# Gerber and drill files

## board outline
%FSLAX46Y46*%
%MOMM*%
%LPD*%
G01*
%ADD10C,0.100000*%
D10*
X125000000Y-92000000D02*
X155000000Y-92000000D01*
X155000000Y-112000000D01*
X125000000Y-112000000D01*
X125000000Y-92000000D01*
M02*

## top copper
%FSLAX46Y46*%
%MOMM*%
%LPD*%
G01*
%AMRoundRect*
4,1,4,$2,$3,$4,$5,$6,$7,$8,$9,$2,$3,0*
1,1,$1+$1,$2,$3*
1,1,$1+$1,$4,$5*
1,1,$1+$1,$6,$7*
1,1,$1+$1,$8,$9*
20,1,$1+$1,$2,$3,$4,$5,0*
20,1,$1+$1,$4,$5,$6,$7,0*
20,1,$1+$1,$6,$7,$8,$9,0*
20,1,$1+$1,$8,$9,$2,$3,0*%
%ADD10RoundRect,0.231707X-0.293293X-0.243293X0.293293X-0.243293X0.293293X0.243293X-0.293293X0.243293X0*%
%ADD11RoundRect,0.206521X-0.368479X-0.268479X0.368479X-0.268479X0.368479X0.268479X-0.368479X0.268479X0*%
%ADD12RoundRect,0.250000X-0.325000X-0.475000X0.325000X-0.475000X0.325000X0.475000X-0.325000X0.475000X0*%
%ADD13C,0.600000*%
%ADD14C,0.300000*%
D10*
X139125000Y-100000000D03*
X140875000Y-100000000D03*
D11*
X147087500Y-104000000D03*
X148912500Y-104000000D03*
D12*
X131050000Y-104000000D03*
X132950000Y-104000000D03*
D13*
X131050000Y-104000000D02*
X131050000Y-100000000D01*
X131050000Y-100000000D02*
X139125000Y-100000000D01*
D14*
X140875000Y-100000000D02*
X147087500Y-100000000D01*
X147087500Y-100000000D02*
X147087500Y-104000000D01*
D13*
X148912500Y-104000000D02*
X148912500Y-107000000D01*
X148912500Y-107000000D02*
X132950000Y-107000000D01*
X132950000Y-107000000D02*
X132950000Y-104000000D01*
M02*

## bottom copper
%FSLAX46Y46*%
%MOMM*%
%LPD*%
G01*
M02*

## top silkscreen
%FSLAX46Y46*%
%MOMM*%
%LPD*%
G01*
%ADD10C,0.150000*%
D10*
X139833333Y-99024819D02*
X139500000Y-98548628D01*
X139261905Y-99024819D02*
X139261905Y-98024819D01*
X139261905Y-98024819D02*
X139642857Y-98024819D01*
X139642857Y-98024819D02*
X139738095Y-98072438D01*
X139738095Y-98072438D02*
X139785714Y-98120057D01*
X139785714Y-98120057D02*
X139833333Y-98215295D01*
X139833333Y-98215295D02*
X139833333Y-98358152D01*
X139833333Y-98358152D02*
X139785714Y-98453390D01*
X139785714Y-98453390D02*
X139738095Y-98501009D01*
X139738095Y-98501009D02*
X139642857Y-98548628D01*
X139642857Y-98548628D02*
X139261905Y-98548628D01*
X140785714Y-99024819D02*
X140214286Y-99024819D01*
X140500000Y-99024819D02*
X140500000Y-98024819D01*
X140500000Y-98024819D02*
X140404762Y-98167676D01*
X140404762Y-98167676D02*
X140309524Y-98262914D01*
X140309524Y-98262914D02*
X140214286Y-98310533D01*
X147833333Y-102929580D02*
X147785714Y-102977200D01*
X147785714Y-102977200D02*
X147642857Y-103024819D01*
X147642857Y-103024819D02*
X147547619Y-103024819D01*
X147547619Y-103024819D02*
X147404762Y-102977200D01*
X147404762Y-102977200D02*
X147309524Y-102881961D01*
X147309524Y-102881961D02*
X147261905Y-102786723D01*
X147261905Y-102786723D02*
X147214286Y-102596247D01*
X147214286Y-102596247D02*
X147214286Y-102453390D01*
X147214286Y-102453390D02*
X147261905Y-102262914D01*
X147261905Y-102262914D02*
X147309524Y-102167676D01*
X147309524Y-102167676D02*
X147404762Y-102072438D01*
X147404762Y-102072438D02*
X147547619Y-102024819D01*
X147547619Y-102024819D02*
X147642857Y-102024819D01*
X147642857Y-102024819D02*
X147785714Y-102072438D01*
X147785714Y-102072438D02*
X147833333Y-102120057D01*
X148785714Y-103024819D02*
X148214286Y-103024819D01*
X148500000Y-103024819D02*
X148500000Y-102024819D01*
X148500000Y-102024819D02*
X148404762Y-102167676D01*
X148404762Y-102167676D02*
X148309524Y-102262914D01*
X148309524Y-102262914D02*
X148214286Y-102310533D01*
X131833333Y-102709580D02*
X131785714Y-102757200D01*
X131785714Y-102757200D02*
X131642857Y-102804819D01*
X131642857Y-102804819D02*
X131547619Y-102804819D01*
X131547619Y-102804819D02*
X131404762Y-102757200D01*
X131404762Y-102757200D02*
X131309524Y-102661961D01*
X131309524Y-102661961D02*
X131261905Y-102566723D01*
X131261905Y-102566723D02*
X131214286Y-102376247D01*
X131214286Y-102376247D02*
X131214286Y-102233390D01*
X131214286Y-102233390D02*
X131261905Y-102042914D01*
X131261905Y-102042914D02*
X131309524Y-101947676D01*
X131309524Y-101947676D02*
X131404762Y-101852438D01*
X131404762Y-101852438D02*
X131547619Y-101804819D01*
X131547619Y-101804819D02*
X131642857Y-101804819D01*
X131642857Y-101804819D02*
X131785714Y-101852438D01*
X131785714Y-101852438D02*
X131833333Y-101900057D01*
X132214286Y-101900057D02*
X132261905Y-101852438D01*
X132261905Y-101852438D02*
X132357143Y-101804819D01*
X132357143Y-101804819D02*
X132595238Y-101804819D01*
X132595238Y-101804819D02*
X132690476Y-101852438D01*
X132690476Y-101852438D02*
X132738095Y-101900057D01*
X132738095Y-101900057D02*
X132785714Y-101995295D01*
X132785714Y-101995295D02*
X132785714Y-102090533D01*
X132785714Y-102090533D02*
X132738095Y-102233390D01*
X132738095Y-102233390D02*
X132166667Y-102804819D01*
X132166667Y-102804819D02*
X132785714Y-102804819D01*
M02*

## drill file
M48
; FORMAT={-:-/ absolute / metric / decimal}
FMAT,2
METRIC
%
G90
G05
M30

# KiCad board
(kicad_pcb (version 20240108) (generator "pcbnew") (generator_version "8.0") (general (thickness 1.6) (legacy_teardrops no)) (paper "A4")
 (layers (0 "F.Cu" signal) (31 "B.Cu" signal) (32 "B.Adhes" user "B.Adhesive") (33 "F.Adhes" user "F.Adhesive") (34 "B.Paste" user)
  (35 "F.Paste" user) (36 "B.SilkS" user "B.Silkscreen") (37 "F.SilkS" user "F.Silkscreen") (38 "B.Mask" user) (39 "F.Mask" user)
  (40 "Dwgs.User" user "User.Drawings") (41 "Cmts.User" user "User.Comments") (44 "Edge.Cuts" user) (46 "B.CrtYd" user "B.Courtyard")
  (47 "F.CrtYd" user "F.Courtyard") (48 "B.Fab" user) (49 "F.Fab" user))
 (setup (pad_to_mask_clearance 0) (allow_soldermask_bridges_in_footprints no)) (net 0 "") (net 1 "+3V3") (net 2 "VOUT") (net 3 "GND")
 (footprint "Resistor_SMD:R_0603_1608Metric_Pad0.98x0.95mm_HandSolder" (layer "F.Cu") (at 140 100 0)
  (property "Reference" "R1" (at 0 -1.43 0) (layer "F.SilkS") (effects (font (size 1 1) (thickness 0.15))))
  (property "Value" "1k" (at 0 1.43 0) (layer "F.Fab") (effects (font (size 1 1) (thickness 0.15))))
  (pad "1" smd roundrect (at -0.875 0 0) (size 1.05 0.95) (layers "F.Cu" "F.Paste" "F.Mask") (roundrect_rratio 0.243902) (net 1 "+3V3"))
  (pad "2" smd roundrect (at 0.875 0 0) (size 1.05 0.95) (layers "F.Cu" "F.Paste" "F.Mask") (roundrect_rratio 0.243902) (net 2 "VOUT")))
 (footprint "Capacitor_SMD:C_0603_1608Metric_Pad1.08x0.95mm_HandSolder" (layer "F.Cu") (at 148 104)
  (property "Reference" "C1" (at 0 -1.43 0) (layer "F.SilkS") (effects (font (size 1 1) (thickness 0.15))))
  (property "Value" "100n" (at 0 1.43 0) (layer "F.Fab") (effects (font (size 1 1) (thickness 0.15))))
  (pad "1" smd roundrect (at -0.9125 0) (size 1.15 0.95) (layers "F.Cu" "F.Paste" "F.Mask") (roundrect_rratio 0.217391) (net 2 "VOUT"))
  (pad "2" smd roundrect (at 0.9125 0) (size 1.15 0.95) (layers "F.Cu" "F.Paste" "F.Mask") (roundrect_rratio 0.217391) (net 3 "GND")))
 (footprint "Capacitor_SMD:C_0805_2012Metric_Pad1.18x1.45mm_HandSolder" (layer "F.Cu") (at 132 104)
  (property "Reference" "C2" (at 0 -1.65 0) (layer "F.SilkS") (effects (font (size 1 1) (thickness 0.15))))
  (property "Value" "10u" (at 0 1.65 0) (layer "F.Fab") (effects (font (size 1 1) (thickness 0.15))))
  (pad "1" smd roundrect (at -0.95 0) (size 1.15 1.45) (layers "F.Cu" "F.Paste" "F.Mask") (roundrect_rratio 0.217391) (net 1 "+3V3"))
  (pad "2" smd roundrect (at 0.95 0) (size 1.15 1.45) (layers "F.Cu" "F.Paste" "F.Mask") (roundrect_rratio 0.217391) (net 3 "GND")))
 (gr_rect (start 125 92) (end 155 112) (stroke (width 0.1) (type default)) (fill none) (layer "Edge.Cuts"))
 (segment (start 131.05 104) (end 131.05 100) (width 0.6) (layer "F.Cu") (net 1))
 (segment (start 131.05 100) (end 139.125 100) (width 0.6) (layer "F.Cu") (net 1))
 (segment (start 140.875 100) (end 147.0875 100) (width 0.3) (layer "F.Cu") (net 2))
 (segment (start 147.0875 100) (end 147.0875 104) (width 0.3) (layer "F.Cu") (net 2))
 (segment (start 148.9125 104) (end 148.9125 107) (width 0.6) (layer "F.Cu") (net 3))
 (segment (start 148.9125 107) (end 132.95 107) (width 0.6) (layer "F.Cu") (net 3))
 (segment (start 132.95 107) (end 132.95 104) (width 0.6) (layer "F.Cu") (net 3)))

